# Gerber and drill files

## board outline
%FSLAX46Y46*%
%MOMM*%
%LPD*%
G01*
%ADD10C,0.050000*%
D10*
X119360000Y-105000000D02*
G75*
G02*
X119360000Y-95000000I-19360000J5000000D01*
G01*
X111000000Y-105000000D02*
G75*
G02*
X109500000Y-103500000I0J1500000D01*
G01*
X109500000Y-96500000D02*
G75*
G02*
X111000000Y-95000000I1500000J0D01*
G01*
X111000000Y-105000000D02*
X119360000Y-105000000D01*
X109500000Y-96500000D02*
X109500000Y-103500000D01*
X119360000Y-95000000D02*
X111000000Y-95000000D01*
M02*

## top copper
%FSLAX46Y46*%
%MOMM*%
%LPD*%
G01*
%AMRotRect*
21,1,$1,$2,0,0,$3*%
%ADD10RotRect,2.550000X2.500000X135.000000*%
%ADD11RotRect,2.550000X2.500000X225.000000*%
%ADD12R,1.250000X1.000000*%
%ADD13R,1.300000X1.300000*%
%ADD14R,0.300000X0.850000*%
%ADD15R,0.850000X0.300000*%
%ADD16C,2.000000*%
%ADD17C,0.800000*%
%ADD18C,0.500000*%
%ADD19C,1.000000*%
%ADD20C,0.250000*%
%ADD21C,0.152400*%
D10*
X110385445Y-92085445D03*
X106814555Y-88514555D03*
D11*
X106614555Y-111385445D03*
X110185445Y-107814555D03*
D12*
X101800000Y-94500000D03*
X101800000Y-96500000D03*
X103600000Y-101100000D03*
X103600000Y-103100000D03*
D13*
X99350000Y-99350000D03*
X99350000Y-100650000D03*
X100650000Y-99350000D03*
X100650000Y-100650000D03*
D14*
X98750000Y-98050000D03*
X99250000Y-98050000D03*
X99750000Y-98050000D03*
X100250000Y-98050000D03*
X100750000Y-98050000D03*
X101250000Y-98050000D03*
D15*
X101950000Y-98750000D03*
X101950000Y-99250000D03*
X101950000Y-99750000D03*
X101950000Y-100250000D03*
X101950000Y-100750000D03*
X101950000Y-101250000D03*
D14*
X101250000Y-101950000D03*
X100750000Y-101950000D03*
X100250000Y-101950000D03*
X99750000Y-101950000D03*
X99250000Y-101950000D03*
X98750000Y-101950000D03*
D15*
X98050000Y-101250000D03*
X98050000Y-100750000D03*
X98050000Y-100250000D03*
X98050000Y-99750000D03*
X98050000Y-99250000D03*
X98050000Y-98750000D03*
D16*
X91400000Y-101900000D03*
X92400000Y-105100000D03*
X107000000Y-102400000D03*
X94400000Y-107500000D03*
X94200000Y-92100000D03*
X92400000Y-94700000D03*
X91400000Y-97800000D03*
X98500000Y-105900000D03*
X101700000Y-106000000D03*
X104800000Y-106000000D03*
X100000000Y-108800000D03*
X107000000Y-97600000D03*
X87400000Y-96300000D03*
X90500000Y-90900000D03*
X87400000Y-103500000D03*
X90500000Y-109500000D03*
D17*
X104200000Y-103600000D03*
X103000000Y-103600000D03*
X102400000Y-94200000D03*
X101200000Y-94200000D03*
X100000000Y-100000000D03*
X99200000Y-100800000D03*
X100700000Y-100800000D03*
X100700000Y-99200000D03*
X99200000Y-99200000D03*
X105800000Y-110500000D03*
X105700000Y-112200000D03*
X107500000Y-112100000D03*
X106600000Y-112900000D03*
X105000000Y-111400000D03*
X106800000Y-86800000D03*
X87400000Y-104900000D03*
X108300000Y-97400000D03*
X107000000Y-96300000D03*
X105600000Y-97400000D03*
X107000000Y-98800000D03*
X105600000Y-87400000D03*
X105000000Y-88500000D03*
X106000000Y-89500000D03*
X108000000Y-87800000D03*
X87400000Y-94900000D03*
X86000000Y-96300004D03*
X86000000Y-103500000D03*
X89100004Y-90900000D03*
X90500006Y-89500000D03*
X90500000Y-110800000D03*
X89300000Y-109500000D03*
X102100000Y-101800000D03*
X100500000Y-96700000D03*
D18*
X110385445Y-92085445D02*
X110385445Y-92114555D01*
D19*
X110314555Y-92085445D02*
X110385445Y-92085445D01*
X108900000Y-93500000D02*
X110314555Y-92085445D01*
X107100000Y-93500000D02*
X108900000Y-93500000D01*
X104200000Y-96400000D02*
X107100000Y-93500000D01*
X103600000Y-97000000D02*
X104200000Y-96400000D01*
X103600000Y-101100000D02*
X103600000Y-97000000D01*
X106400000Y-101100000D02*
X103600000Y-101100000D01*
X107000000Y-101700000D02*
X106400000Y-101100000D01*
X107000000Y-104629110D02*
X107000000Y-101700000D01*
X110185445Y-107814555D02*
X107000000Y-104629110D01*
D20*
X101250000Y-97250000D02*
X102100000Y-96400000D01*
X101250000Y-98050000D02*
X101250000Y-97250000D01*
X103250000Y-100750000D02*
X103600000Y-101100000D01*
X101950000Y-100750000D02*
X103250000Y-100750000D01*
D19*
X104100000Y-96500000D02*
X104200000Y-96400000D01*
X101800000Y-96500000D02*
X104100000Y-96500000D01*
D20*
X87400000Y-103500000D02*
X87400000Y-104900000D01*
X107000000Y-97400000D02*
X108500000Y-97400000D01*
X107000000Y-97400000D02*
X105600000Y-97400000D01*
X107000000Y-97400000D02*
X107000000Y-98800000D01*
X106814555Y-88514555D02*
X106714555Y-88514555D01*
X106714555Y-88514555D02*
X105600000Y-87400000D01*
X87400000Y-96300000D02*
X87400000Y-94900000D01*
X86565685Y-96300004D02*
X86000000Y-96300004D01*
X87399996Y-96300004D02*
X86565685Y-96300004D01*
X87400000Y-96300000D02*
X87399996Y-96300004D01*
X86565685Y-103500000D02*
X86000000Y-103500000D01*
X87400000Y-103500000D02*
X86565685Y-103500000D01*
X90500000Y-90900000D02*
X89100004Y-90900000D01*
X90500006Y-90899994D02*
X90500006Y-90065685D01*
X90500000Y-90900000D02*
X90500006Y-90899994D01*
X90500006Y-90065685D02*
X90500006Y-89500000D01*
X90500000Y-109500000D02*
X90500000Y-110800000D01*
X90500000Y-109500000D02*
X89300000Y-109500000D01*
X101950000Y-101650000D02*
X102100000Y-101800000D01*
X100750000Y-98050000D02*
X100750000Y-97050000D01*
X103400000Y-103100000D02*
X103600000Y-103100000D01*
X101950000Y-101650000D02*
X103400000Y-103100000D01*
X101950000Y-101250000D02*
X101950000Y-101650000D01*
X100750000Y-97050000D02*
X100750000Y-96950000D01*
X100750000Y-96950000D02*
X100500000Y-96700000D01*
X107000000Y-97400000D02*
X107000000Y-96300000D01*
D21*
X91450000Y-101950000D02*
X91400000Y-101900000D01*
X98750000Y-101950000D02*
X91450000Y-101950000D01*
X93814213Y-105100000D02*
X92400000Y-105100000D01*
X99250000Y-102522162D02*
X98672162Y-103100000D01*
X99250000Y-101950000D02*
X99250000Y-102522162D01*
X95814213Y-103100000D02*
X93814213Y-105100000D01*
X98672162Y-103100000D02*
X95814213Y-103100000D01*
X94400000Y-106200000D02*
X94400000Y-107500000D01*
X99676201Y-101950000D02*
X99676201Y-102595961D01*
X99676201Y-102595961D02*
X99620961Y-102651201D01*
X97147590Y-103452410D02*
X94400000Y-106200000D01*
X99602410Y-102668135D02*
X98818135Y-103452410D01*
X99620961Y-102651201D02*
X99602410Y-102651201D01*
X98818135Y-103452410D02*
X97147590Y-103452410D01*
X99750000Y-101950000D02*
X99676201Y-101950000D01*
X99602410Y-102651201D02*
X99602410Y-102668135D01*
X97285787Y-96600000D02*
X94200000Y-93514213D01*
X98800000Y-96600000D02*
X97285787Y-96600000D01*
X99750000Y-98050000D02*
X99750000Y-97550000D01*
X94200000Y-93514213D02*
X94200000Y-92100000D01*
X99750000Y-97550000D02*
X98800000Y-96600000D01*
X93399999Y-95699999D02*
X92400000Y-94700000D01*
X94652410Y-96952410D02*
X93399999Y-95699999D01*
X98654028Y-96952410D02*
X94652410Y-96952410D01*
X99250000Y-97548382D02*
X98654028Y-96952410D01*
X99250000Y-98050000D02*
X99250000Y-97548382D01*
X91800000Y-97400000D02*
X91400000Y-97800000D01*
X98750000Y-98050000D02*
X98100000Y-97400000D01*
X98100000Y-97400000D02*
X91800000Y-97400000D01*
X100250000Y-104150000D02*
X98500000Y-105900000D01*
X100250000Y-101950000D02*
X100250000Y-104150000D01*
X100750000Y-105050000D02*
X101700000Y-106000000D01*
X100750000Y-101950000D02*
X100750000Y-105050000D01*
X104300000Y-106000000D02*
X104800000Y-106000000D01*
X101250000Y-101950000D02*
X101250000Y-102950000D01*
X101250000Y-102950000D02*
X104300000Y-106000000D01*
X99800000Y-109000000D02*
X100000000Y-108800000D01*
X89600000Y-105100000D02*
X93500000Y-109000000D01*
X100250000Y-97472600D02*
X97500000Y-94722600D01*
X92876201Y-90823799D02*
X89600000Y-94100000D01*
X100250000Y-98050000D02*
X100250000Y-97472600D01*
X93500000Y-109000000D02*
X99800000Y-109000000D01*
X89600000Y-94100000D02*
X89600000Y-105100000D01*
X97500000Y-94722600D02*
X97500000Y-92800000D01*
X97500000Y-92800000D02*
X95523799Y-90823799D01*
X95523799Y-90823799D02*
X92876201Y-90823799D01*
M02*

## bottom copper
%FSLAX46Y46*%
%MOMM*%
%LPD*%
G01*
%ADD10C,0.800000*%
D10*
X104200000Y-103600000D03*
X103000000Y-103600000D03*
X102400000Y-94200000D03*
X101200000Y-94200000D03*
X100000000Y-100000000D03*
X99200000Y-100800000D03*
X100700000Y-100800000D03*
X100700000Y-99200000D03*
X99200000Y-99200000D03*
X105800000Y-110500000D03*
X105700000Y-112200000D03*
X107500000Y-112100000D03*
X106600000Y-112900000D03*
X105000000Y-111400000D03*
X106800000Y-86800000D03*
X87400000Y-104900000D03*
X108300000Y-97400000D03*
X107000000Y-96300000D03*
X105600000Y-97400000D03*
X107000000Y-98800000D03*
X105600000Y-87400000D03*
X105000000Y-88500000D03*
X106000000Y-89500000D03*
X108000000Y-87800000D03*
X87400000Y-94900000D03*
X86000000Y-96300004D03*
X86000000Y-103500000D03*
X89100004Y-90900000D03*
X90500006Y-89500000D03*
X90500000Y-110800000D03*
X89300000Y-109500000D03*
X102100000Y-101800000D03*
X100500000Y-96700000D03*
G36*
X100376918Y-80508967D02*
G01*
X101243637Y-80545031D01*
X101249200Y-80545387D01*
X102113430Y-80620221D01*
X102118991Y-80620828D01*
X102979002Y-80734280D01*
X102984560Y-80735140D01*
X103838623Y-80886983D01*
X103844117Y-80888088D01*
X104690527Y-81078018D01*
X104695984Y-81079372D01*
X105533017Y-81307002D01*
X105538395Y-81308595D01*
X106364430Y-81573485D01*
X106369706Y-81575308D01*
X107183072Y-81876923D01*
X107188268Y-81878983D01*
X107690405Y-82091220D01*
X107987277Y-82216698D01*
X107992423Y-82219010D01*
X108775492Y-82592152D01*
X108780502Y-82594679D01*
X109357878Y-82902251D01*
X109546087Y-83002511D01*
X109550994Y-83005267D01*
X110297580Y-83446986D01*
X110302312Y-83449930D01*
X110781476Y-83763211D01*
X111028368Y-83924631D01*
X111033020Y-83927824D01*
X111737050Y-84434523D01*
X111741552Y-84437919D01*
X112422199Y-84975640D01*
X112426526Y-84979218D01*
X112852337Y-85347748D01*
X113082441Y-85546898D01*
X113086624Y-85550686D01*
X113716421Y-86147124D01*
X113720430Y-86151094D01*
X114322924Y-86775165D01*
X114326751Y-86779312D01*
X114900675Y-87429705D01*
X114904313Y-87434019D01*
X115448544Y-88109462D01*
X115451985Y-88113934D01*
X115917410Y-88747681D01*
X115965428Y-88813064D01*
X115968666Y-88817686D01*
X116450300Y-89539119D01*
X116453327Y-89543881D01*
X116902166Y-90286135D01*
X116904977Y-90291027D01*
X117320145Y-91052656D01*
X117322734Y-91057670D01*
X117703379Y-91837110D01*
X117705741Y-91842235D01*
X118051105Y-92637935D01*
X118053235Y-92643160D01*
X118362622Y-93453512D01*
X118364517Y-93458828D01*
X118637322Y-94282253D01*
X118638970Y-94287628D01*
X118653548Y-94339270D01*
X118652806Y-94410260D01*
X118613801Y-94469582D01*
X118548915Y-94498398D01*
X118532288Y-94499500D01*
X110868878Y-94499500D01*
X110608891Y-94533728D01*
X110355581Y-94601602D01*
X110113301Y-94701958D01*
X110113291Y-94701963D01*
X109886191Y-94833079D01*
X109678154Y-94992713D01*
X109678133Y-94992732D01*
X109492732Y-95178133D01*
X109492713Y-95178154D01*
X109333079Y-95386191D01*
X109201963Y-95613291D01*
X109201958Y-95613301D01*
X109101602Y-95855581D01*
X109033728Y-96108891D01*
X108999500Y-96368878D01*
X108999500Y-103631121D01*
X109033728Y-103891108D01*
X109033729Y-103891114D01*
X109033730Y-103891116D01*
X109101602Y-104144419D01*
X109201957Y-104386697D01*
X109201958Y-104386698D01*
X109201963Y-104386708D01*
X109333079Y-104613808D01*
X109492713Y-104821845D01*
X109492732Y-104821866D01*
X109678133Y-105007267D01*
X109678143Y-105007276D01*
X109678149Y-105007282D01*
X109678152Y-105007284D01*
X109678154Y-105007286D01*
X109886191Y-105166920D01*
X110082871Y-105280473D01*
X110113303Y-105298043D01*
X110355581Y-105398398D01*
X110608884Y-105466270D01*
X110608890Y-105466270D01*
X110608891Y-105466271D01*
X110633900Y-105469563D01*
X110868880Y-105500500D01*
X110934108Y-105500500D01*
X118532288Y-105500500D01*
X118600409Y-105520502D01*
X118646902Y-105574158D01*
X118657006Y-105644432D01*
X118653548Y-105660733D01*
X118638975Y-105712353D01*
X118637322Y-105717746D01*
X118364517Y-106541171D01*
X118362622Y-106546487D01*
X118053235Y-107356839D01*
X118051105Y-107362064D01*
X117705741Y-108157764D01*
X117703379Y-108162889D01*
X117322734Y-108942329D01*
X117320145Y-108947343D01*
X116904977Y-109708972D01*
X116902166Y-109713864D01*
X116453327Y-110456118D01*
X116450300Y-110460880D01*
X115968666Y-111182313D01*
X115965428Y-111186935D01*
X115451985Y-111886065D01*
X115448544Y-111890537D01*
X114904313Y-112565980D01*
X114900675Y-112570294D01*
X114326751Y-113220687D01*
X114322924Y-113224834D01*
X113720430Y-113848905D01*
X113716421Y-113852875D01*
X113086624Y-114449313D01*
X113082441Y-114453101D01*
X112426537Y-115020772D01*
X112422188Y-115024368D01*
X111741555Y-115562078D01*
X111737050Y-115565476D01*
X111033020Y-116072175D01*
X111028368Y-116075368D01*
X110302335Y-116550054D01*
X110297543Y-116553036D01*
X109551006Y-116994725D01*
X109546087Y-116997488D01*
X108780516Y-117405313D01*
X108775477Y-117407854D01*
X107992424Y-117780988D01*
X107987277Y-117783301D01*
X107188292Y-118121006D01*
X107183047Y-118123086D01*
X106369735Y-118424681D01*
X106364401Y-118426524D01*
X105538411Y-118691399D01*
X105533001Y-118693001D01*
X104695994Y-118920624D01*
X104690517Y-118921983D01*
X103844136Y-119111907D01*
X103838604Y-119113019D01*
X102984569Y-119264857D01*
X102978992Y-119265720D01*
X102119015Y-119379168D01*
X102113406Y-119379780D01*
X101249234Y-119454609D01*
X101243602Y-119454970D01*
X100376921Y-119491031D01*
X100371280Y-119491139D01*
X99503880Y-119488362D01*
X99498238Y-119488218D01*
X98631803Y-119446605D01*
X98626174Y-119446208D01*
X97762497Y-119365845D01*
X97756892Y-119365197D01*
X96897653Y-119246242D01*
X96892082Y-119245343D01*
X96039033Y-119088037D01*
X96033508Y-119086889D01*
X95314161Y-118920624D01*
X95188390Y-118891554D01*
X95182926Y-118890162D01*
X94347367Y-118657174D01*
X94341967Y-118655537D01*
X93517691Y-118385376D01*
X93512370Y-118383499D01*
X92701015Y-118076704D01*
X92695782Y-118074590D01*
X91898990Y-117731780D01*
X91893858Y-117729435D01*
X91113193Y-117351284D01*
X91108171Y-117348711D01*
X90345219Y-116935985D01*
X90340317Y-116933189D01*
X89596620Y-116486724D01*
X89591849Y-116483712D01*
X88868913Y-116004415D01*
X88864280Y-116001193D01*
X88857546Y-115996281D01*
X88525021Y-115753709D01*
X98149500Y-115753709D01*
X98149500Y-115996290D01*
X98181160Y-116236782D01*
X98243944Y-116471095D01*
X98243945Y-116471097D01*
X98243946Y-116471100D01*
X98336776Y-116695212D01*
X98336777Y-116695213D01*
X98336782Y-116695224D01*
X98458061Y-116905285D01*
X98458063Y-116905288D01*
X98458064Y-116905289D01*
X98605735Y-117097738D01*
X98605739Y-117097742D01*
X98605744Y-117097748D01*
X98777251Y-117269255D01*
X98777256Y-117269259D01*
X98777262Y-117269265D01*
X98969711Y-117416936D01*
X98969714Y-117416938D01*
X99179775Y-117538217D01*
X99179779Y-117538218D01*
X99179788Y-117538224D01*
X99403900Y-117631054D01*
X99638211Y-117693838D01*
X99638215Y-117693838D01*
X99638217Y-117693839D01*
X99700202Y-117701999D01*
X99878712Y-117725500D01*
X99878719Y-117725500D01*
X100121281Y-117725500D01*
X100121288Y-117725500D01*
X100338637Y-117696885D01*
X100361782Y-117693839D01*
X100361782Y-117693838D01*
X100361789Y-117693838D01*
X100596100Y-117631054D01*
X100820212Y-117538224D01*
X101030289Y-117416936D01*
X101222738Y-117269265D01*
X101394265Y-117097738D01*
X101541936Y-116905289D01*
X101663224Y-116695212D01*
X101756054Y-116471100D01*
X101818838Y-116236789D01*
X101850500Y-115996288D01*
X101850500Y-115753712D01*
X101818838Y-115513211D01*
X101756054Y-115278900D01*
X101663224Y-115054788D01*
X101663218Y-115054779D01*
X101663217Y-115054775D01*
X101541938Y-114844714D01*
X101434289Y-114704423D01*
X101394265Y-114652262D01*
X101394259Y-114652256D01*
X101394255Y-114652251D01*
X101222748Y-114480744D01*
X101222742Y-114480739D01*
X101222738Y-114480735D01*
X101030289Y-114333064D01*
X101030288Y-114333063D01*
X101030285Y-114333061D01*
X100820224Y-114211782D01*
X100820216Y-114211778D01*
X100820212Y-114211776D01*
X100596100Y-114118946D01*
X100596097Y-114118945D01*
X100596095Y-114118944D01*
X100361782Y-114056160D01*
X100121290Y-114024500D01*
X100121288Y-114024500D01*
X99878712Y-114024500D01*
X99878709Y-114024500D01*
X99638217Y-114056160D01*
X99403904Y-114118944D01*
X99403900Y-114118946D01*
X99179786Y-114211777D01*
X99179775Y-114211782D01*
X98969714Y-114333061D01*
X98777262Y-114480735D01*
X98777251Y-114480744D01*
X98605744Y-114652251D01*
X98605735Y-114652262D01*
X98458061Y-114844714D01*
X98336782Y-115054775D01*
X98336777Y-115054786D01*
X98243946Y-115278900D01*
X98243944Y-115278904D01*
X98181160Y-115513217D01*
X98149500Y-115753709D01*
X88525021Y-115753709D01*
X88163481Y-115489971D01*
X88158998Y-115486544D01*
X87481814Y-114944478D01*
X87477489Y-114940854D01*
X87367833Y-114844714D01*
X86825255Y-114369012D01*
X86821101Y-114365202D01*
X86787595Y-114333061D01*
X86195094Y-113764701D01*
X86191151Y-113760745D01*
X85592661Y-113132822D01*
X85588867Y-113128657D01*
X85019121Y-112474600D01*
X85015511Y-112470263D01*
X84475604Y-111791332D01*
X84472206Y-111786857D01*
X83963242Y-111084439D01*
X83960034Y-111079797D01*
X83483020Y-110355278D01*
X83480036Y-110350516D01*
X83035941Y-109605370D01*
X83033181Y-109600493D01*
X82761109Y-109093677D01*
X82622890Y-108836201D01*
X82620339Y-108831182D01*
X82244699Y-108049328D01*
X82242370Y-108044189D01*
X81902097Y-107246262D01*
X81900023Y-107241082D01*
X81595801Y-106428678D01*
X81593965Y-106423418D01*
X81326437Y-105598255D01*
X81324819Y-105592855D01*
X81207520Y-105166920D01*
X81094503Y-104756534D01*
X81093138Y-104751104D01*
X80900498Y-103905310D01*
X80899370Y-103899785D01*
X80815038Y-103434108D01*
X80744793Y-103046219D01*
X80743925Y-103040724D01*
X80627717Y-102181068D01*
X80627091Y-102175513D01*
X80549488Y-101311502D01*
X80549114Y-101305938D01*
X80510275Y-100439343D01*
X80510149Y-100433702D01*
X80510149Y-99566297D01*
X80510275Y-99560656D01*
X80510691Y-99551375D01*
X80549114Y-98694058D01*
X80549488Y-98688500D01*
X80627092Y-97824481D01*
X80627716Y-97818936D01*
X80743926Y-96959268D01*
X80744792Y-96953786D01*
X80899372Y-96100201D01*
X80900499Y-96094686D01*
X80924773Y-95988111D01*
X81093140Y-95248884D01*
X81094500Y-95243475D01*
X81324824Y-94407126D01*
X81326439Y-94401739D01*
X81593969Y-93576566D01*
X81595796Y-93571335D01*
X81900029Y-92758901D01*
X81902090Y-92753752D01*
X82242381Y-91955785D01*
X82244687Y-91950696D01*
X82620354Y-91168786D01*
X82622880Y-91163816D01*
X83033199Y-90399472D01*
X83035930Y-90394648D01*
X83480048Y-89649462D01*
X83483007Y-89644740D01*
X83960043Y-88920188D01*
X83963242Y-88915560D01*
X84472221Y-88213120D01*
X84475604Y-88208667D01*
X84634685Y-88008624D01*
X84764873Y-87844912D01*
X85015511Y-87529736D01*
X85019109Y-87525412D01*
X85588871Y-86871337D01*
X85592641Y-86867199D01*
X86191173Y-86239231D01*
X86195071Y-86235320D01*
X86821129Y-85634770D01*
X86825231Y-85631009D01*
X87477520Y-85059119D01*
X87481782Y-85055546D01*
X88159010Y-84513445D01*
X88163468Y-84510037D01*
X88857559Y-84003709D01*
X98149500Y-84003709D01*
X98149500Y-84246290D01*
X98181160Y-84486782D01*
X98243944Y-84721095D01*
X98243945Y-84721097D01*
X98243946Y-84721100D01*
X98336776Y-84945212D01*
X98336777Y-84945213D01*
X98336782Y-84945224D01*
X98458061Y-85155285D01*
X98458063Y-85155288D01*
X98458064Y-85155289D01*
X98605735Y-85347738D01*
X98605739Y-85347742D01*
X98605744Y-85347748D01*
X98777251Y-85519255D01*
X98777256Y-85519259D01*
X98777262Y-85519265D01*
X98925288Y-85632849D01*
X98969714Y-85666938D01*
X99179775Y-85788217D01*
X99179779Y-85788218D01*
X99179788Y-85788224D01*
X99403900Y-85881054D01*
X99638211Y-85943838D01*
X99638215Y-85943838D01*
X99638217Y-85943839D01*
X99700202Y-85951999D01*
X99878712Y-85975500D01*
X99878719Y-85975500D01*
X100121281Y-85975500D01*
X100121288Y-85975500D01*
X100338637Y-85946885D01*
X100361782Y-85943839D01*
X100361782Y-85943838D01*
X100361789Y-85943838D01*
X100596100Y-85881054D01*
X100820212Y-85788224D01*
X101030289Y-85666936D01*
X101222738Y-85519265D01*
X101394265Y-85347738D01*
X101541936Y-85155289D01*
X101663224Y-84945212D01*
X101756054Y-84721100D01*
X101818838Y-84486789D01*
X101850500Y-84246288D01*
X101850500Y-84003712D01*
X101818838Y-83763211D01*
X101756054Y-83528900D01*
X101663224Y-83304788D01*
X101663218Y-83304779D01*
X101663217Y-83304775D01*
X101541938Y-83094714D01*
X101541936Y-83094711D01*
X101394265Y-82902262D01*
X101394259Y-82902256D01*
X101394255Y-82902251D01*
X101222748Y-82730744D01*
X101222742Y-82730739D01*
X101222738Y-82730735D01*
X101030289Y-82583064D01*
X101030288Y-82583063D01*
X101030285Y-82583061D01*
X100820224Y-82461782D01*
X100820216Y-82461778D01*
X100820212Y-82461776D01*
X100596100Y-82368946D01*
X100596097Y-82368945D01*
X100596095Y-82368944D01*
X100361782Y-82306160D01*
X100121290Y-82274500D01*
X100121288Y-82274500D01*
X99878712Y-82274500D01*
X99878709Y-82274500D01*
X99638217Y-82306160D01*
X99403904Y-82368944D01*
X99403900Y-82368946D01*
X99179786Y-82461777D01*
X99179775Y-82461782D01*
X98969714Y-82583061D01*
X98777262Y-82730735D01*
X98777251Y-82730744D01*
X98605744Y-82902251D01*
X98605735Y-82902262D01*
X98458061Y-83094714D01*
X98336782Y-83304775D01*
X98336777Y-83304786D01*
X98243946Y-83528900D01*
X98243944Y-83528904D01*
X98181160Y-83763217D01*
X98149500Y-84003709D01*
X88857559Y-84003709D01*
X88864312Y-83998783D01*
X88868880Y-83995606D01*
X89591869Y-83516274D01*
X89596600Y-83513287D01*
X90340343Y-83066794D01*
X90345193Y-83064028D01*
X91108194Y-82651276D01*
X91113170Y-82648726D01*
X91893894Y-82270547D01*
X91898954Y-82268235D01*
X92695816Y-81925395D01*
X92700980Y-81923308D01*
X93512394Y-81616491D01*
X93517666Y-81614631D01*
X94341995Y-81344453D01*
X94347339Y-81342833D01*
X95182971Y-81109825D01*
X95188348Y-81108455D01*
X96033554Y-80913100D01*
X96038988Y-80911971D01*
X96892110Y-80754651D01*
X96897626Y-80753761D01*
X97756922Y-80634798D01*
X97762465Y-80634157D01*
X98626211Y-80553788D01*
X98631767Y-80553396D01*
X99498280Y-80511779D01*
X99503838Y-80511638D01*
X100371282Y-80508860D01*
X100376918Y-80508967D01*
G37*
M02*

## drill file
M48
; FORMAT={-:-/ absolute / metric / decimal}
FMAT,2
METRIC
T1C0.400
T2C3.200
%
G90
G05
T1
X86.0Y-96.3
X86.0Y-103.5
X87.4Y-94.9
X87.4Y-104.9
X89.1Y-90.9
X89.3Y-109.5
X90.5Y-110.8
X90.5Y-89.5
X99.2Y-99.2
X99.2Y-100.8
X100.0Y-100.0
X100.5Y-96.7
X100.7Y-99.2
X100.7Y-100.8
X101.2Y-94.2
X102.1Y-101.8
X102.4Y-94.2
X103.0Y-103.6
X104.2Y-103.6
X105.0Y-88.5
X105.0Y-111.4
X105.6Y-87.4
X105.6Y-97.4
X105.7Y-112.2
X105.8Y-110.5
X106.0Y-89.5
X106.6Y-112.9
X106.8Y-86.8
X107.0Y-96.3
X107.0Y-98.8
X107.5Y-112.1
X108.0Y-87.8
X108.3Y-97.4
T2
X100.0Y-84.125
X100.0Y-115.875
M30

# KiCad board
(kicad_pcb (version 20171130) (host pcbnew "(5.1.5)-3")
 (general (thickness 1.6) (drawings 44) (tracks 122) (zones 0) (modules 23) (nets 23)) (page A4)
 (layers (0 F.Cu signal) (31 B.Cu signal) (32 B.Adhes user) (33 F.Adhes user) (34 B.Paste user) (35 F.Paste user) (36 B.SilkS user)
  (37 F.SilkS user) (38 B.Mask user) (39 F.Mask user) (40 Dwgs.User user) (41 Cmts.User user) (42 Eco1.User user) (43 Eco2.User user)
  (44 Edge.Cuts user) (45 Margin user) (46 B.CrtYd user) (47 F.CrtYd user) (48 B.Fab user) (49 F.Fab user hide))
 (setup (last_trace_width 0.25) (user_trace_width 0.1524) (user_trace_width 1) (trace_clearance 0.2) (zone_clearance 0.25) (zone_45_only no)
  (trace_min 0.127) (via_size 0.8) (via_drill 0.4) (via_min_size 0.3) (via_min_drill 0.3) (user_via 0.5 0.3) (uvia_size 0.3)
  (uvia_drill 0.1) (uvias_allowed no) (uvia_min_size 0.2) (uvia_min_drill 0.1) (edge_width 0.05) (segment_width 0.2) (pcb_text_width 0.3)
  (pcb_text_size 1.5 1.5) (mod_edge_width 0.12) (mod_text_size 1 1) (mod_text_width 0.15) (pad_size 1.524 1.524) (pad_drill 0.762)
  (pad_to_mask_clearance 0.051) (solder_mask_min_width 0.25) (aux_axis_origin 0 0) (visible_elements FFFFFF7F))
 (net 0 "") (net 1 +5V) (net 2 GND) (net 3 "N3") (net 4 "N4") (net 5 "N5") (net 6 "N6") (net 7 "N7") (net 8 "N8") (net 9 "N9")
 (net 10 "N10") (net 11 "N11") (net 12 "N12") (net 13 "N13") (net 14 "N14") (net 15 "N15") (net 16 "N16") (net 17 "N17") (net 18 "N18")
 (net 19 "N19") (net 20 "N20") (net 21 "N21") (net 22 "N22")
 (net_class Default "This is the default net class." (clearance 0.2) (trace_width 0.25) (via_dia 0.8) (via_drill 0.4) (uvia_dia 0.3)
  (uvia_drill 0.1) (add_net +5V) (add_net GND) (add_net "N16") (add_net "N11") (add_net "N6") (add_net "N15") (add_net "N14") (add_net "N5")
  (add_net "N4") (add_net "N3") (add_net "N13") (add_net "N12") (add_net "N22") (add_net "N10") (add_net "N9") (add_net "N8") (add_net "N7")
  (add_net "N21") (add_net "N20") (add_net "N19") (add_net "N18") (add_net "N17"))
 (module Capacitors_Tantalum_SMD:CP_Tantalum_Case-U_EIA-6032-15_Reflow (layer F.Cu) (at 108.6 90.3 135)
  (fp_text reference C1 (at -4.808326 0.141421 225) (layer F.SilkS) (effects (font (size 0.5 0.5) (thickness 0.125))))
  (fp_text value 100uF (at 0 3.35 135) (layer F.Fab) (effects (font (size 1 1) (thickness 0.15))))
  (pad 1 smd rect (at -2.525 0 135) (size 2.55 2.5) (layers F.Cu F.Paste F.Mask) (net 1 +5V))
  (pad 2 smd rect (at 2.525 0 135) (size 2.55 2.5) (layers F.Cu F.Paste F.Mask) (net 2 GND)))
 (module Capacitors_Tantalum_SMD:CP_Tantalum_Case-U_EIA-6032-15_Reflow (layer F.Cu) (at 108.4 109.6 225)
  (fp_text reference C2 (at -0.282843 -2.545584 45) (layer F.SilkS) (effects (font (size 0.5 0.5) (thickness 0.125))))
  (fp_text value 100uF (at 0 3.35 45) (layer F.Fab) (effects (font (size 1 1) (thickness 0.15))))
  (pad 2 smd rect (at 2.525 0 225) (size 2.55 2.5) (layers F.Cu F.Paste F.Mask) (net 2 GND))
  (pad 1 smd rect (at -2.525 0 225) (size 2.55 2.5) (layers F.Cu F.Paste F.Mask) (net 1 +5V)))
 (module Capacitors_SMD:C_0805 (layer F.Cu) (at 101.8 95.5 90)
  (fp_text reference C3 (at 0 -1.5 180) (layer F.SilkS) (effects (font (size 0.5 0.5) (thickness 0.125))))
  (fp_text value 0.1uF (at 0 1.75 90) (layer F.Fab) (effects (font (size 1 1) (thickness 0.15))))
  (pad 2 smd rect (at 1 0 90) (size 1 1.25) (layers F.Cu F.Paste F.Mask) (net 2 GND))
  (pad 1 smd rect (at -1 0 90) (size 1 1.25) (layers F.Cu F.Paste F.Mask) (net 1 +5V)))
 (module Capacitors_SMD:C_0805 (layer F.Cu) (at 103.6 102.1 270)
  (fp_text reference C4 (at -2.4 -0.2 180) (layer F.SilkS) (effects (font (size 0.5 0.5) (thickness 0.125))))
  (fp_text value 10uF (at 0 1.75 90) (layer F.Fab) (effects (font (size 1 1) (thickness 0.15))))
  (pad 1 smd rect (at -1 0 270) (size 1 1.25) (layers F.Cu F.Paste F.Mask) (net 1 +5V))
  (pad 2 smd rect (at 1 0 270) (size 1 1.25) (layers F.Cu F.Paste F.Mask) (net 2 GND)))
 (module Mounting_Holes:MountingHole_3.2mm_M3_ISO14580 (layer F.Cu) (at 100 84.125)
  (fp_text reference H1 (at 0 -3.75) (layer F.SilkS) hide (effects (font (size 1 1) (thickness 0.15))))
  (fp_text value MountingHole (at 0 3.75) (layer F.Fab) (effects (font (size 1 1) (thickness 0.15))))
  (pad 1 np_thru_hole circle (at 0 0) (size 3.2 3.2) (drill 3.2) (layers *.Cu *.Mask)))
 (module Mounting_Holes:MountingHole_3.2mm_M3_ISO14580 (layer F.Cu) (at 100 115.875)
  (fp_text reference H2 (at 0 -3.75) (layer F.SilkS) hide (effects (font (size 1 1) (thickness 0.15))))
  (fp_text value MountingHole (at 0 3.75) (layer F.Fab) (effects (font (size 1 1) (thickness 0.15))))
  (pad 1 np_thru_hole circle (at 0 0) (size 3.2 3.2) (drill 3.2) (layers *.Cu *.Mask)))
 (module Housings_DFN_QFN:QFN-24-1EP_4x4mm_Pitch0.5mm (layer F.Cu) (at 100 100) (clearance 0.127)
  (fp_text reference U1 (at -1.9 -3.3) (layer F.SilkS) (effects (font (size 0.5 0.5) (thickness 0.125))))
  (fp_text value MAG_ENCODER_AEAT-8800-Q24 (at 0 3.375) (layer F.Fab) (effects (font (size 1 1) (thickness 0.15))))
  (pad 25 smd rect (at -0.65 -0.65) (size 1.3 1.3) (layers F.Cu F.Paste F.Mask) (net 2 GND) (solder_paste_margin_ratio -0.2))
  (pad 25 smd rect (at -0.65 0.65) (size 1.3 1.3) (layers F.Cu F.Paste F.Mask) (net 2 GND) (solder_paste_margin_ratio -0.2))
  (pad 25 smd rect (at 0.65 -0.65) (size 1.3 1.3) (layers F.Cu F.Paste F.Mask) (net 2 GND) (solder_paste_margin_ratio -0.2))
  (pad 25 smd rect (at 0.65 0.65) (size 1.3 1.3) (layers F.Cu F.Paste F.Mask) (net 2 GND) (solder_paste_margin_ratio -0.2))
  (pad 24 smd rect (at -1.25 -1.95 90) (size 0.85 0.3) (layers F.Cu F.Paste F.Mask) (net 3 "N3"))
  (pad 23 smd rect (at -0.75 -1.95 90) (size 0.85 0.3) (layers F.Cu F.Paste F.Mask) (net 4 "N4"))
  (pad 22 smd rect (at -0.25 -1.95 90) (size 0.85 0.3) (layers F.Cu F.Paste F.Mask) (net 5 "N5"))
  (pad 21 smd rect (at 0.25 -1.95 90) (size 0.85 0.3) (layers F.Cu F.Paste F.Mask) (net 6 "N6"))
  (pad 20 smd rect (at 0.75 -1.95 90) (size 0.85 0.3) (layers F.Cu F.Paste F.Mask) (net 2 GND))
  (pad 19 smd rect (at 1.25 -1.95 90) (size 0.85 0.3) (layers F.Cu F.Paste F.Mask) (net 1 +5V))
  (pad 18 smd rect (at 1.95 -1.25) (size 0.85 0.3) (layers F.Cu F.Paste F.Mask) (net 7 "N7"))
  (pad 17 smd rect (at 1.95 -0.75) (size 0.85 0.3) (layers F.Cu F.Paste F.Mask) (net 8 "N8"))
  (pad 16 smd rect (at 1.95 -0.25) (size 0.85 0.3) (layers F.Cu F.Paste F.Mask) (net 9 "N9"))
  (pad 15 smd rect (at 1.95 0.25) (size 0.85 0.3) (layers F.Cu F.Paste F.Mask) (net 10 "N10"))
  (pad 14 smd rect (at 1.95 0.75) (size 0.85 0.3) (layers F.Cu F.Paste F.Mask) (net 1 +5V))
  (pad 13 smd rect (at 1.95 1.25) (size 0.85 0.3) (layers F.Cu F.Paste F.Mask) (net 2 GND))
  (pad 12 smd rect (at 1.25 1.95 90) (size 0.85 0.3) (layers F.Cu F.Paste F.Mask) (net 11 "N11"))
  (pad 11 smd rect (at 0.75 1.95 90) (size 0.85 0.3) (layers F.Cu F.Paste F.Mask) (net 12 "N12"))
  (pad 10 smd rect (at 0.25 1.95 90) (size 0.85 0.3) (layers F.Cu F.Paste F.Mask) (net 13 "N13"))
  (pad 9 smd rect (at -0.25 1.95 90) (size 0.85 0.3) (layers F.Cu F.Paste F.Mask) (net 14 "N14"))
  (pad 8 smd rect (at -0.75 1.95 90) (size 0.85 0.3) (layers F.Cu F.Paste F.Mask) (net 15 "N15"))
  (pad 7 smd rect (at -1.25 1.95 90) (size 0.85 0.3) (layers F.Cu F.Paste F.Mask) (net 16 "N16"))
  (pad 6 smd rect (at -1.95 1.25) (size 0.85 0.3) (layers F.Cu F.Paste F.Mask) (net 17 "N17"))
  (pad 5 smd rect (at -1.95 0.75) (size 0.85 0.3) (layers F.Cu F.Paste F.Mask) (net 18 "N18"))
  (pad 4 smd rect (at -1.95 0.25) (size 0.85 0.3) (layers F.Cu F.Paste F.Mask) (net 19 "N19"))
  (pad 3 smd rect (at -1.95 -0.25) (size 0.85 0.3) (layers F.Cu F.Paste F.Mask) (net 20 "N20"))
  (pad 2 smd rect (at -1.95 -0.75) (size 0.85 0.3) (layers F.Cu F.Paste F.Mask) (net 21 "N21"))
  (pad 1 smd rect (at -1.95 -1.25) (size 0.85 0.3) (layers F.Cu F.Paste F.Mask) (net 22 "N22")))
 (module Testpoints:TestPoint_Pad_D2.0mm (layer F.Cu) (at 91.4 101.9)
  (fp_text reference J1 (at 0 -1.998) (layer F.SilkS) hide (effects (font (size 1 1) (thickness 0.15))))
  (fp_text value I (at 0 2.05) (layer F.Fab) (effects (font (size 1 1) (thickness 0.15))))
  (pad 1 smd circle (at 0 0) (size 2 2) (layers F.Cu F.Mask) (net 16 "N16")))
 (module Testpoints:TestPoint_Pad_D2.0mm (layer F.Cu) (at 92.4 105.1)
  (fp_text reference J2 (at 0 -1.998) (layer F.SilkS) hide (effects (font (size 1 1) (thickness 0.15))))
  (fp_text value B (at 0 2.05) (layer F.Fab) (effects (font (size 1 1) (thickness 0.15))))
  (pad 1 smd circle (at 0 0) (size 2 2) (layers F.Cu F.Mask) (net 15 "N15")))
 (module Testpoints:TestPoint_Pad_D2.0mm (layer F.Cu) (at 107 102.4)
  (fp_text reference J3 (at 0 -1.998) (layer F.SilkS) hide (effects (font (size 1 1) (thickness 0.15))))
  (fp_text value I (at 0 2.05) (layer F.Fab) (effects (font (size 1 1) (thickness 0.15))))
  (pad 1 smd circle (at 0 0) (size 2 2) (layers F.Cu F.Mask) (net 1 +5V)))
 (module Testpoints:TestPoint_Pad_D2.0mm (layer F.Cu) (at 94.4 107.5)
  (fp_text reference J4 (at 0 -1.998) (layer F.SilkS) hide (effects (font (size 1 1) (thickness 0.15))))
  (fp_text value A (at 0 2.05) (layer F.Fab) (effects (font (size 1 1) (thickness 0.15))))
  (pad 1 smd circle (at 0 0) (size 2 2) (layers F.Cu F.Mask) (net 14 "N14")))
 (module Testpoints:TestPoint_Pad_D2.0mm (layer F.Cu) (at 94.2 92.1)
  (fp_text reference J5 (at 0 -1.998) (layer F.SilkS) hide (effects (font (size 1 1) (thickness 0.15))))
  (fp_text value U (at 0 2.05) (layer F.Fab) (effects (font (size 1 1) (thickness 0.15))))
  (pad 1 smd circle (at 0 0) (size 2 2) (layers F.Cu F.Mask) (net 5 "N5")))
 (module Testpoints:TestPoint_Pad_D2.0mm (layer F.Cu) (at 92.4 94.7)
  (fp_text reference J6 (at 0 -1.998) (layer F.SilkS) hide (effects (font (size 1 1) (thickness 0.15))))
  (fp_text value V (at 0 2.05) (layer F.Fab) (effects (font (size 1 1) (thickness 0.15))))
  (pad 1 smd circle (at 0 0) (size 2 2) (layers F.Cu F.Mask) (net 4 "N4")))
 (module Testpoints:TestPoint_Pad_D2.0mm (layer F.Cu) (at 91.4 97.8)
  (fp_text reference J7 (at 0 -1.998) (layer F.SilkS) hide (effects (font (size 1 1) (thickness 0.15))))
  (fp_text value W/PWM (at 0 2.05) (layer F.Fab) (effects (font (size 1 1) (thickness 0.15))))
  (pad 1 smd circle (at 0 0) (size 2 2) (layers F.Cu F.Mask) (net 3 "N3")))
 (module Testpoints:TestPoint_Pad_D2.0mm (layer F.Cu) (at 98.5 105.9)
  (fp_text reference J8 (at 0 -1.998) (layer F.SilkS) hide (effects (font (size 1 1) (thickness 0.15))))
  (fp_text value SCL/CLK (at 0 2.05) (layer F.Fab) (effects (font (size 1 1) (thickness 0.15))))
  (pad 1 smd circle (at 0 0) (size 2 2) (layers F.Cu F.Mask) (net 13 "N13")))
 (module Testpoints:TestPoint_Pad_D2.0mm (layer F.Cu) (at 101.7 106)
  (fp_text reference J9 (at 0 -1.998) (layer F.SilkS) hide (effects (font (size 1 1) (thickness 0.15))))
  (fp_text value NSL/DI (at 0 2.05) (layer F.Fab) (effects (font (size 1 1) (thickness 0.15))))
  (pad 1 smd circle (at 0 0) (size 2 2) (layers F.Cu F.Mask) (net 12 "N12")))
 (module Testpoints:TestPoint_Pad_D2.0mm (layer F.Cu) (at 104.8 106)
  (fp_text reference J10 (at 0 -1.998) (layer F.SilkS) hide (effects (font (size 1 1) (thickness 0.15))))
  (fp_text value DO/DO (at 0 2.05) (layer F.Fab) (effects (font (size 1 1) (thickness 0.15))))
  (pad 1 smd circle (at 0 0) (size 2 2) (layers F.Cu F.Mask) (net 11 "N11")))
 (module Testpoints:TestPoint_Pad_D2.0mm (layer F.Cu) (at 100 108.8)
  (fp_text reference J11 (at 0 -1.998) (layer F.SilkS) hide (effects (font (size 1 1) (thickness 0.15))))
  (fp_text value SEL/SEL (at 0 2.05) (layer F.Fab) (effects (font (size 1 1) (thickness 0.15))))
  (pad 1 smd circle (at 0 0) (size 2 2) (layers F.Cu F.Mask) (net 6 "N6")))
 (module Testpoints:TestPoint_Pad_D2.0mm (layer F.Cu) (at 107 97.6)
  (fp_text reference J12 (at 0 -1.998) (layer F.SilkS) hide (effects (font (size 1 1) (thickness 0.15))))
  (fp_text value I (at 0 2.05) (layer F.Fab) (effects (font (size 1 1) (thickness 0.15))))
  (pad 1 smd circle (at 0 0) (size 2 2) (layers F.Cu F.Mask) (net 2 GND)))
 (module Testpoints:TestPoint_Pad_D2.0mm (layer F.Cu) (at 87.4 96.3)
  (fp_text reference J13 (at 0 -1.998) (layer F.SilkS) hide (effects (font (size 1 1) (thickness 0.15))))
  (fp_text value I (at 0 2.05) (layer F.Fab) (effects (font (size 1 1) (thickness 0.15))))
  (pad 1 smd circle (at 0 0) (size 2 2) (layers F.Cu F.Mask) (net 2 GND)))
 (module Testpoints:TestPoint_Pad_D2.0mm (layer F.Cu) (at 90.5 90.9)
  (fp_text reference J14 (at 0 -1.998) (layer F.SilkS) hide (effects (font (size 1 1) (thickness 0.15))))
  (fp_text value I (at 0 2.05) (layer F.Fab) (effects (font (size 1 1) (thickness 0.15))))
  (pad 1 smd circle (at 0 0) (size 2 2) (layers F.Cu F.Mask) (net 2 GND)))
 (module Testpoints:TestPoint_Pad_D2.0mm (layer F.Cu) (at 87.4 103.5)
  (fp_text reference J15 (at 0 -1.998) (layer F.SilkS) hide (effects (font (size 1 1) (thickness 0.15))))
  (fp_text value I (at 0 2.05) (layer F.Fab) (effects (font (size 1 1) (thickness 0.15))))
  (pad 1 smd circle (at 0 0) (size 2 2) (layers F.Cu F.Mask) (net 2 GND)))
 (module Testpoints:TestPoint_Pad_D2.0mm (layer F.Cu) (at 90.5 109.5)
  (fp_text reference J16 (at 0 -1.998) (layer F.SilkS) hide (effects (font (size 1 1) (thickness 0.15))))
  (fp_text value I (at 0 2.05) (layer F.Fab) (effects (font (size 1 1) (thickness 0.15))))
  (pad 1 smd circle (at 0 0) (size 2 2) (layers F.Cu F.Mask) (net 2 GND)))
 (gr_arc (start 100 100) (end 119.36 95) (angle -331.0379313) (layer Edge.Cuts) (width 0.05))
 (gr_arc (start 111 103.5) (end 109.5 103.5) (angle -90) (layer Edge.Cuts) (width 0.05))
 (gr_arc (start 111 96.5) (end 111 95) (angle -90) (layer Edge.Cuts) (width 0.05))
 (gr_line (start 111 105) (end 119.36 105) (layer Edge.Cuts) (width 0.05))
 (gr_line (start 109.5 96.5) (end 109.5 103.5) (layer Edge.Cuts) (width 0.05))
 (gr_line (start 119.36 95) (end 111 95) (layer Edge.Cuts) (width 0.05))
 (via (at 104.2 103.6) (size 0.8) (drill 0.4) (layers F.Cu B.Cu) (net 2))
 (via (at 103 103.6) (size 0.8) (drill 0.4) (layers F.Cu B.Cu) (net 2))
 (via (at 102.4 94.2) (size 0.8) (drill 0.4) (layers F.Cu B.Cu) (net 2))
 (via (at 101.2 94.2) (size 0.8) (drill 0.4) (layers F.Cu B.Cu) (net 2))
 (via (at 100 100) (size 0.8) (drill 0.4) (layers F.Cu B.Cu) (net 2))
 (via (at 99.2 100.8) (size 0.8) (drill 0.4) (layers F.Cu B.Cu) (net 2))
 (via (at 100.7 100.8) (size 0.8) (drill 0.4) (layers F.Cu B.Cu) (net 2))
 (via (at 100.7 99.2) (size 0.8) (drill 0.4) (layers F.Cu B.Cu) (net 2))
 (via (at 99.2 99.2) (size 0.8) (drill 0.4) (layers F.Cu B.Cu) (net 2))
 (segment (start 110.385445 92.085445) (end 110.385445 92.114555) (width 0.5) (layer F.Cu) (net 1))
 (segment (start 110.314555 92.085445) (end 110.385445 92.085445) (width 1) (layer F.Cu) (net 1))
 (segment (start 108.9 93.5) (end 110.314555 92.085445) (width 1) (layer F.Cu) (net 1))
 (segment (start 107.1 93.5) (end 108.9 93.5) (width 1) (layer F.Cu) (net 1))
 (segment (start 104.2 96.4) (end 107.1 93.5) (width 1) (layer F.Cu) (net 1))
 (segment (start 103.6 97) (end 104.2 96.4) (width 1) (layer F.Cu) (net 1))
 (segment (start 103.6 101.1) (end 103.6 97) (width 1) (layer F.Cu) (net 1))
 (segment (start 106.4 101.1) (end 103.6 101.1) (width 1) (layer F.Cu) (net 1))
 (segment (start 107 101.7) (end 106.4 101.1) (width 1) (layer F.Cu) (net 1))
 (segment (start 107 104.62911) (end 107 101.7) (width 1) (layer F.Cu) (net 1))
 (segment (start 110.185445 107.814555) (end 107 104.62911) (width 1) (layer F.Cu) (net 1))
 (segment (start 101.25 97.25) (end 102.1 96.4) (width 0.25) (layer F.Cu) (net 1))
 (segment (start 101.25 98.05) (end 101.25 97.25) (width 0.25) (layer F.Cu) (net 1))
 (segment (start 103.25 100.75) (end 103.6 101.1) (width 0.25) (layer F.Cu) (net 1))
 (segment (start 101.95 100.75) (end 103.25 100.75) (width 0.25) (layer F.Cu) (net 1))
 (segment (start 104.1 96.5) (end 104.2 96.4) (width 1) (layer F.Cu) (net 1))
 (segment (start 101.8 96.5) (end 104.1 96.5) (width 1) (layer F.Cu) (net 1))
 (via (at 105.8 110.5) (size 0.8) (drill 0.4) (layers F.Cu B.Cu) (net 2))
 (via (at 105.7 112.2) (size 0.8) (drill 0.4) (layers F.Cu B.Cu) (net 2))
 (via (at 107.5 112.1) (size 0.8) (drill 0.4) (layers F.Cu B.Cu) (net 2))
 (via (at 106.6 112.9) (size 0.8) (drill 0.4) (layers F.Cu B.Cu) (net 2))
 (via (at 105 111.4) (size 0.8) (drill 0.4) (layers F.Cu B.Cu) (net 2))
 (via (at 106.8 86.8) (size 0.8) (drill 0.4) (layers F.Cu B.Cu) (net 2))
 (via (at 87.4 104.9) (size 0.8) (drill 0.4) (layers F.Cu B.Cu) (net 2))
 (segment (start 87.4 103.5) (end 87.4 104.9) (width 0.25) (layer F.Cu) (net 2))
 (via (at 108.3 97.4) (size 0.8) (drill 0.4) (layers F.Cu B.Cu) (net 2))
 (segment (start 107 97.4) (end 108.5 97.4) (width 0.25) (layer F.Cu) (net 2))
 (via (at 107 96.3) (size 0.8) (drill 0.4) (layers F.Cu B.Cu) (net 2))
 (via (at 105.6 97.4) (size 0.8) (drill 0.4) (layers F.Cu B.Cu) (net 2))
 (segment (start 107 97.4) (end 105.6 97.4) (width 0.25) (layer F.Cu) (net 2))
 (via (at 107 98.8) (size 0.8) (drill 0.4) (layers F.Cu B.Cu) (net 2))
 (segment (start 107 97.4) (end 107 98.8) (width 0.25) (layer F.Cu) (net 2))
 (via (at 105.6 87.4) (size 0.8) (drill 0.4) (layers F.Cu B.Cu) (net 2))
 (segment (start 106.814555 88.514555) (end 106.714555 88.514555) (width 0.25) (layer F.Cu) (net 2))
 (segment (start 106.714555 88.514555) (end 105.6 87.4) (width 0.25) (layer F.Cu) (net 2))
 (via (at 105 88.5) (size 0.8) (drill 0.4) (layers F.Cu B.Cu) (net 2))
 (via (at 106 89.5) (size 0.8) (drill 0.4) (layers F.Cu B.Cu) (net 2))
 (via (at 108 87.8) (size 0.8) (drill 0.4) (layers F.Cu B.Cu) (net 2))
 (via (at 87.4 94.9) (size 0.8) (drill 0.4) (layers F.Cu B.Cu) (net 2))
 (segment (start 87.4 96.3) (end 87.4 94.9) (width 0.25) (layer F.Cu) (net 2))
 (via (at 86 96.300004) (size 0.8) (drill 0.4) (layers F.Cu B.Cu) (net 2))
 (segment (start 86.565685 96.300004) (end 86 96.300004) (width 0.25) (layer F.Cu) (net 2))
 (segment (start 87.399996 96.300004) (end 86.565685 96.300004) (width 0.25) (layer F.Cu) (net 2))
 (segment (start 87.4 96.3) (end 87.399996 96.300004) (width 0.25) (layer F.Cu) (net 2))
 (segment (start 86.565685 103.5) (end 86 103.5) (width 0.25) (layer F.Cu) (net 2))
 (via (at 86 103.5) (size 0.8) (drill 0.4) (layers F.Cu B.Cu) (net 2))
 (segment (start 87.4 103.5) (end 86.565685 103.5) (width 0.25) (layer F.Cu) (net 2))
 (via (at 89.100004 90.9) (size 0.8) (drill 0.4) (layers F.Cu B.Cu) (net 2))
 (segment (start 90.5 90.9) (end 89.100004 90.9) (width 0.25) (layer F.Cu) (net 2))
 (via (at 90.500006 89.5) (size 0.8) (drill 0.4) (layers F.Cu B.Cu) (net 2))
 (segment (start 90.500006 90.899994) (end 90.500006 90.065685) (width 0.25) (layer F.Cu) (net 2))
 (segment (start 90.5 90.9) (end 90.500006 90.899994) (width 0.25) (layer F.Cu) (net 2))
 (segment (start 90.500006 90.065685) (end 90.500006 89.5) (width 0.25) (layer F.Cu) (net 2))
 (via (at 90.5 110.8) (size 0.8) (drill 0.4) (layers F.Cu B.Cu) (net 2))
 (segment (start 90.5 109.5) (end 90.5 110.8) (width 0.25) (layer F.Cu) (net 2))
 (via (at 89.3 109.5) (size 0.8) (drill 0.4) (layers F.Cu B.Cu) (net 2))
 (segment (start 90.5 109.5) (end 89.3 109.5) (width 0.25) (layer F.Cu) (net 2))
 (via (at 102.1 101.8) (size 0.8) (drill 0.4) (layers F.Cu B.Cu) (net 2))
 (segment (start 101.95 101.65) (end 102.1 101.8) (width 0.25) (layer F.Cu) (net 2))
 (segment (start 100.75 98.05) (end 100.75 97.05) (width 0.25) (layer F.Cu) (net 2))
 (segment (start 103.4 103.1) (end 103.6 103.1) (width 0.25) (layer F.Cu) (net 2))
 (segment (start 101.95 101.65) (end 103.4 103.1) (width 0.25) (layer F.Cu) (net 2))
 (segment (start 101.95 101.25) (end 101.95 101.65) (width 0.25) (layer F.Cu) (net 2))
 (via (at 100.5 96.7) (size 0.8) (drill 0.4) (layers F.Cu B.Cu) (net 2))
 (segment (start 100.75 97.05) (end 100.75 96.95) (width 0.25) (layer F.Cu) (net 2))
 (segment (start 100.75 96.95) (end 100.5 96.7) (width 0.25) (layer F.Cu) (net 2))
 (segment (start 107 97.4) (end 107 96.3) (width 0.25) (layer F.Cu) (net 2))
 (segment (start 91.45 101.95) (end 91.4 101.9) (width 0.1524) (layer F.Cu) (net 16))
 (segment (start 98.75 101.95) (end 91.45 101.95) (width 0.1524) (layer F.Cu) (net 16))
 (segment (start 93.814213 105.1) (end 92.4 105.1) (width 0.1524) (layer F.Cu) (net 15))
 (segment (start 99.25 102.522162) (end 98.672162 103.1) (width 0.1524) (layer F.Cu) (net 15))
 (segment (start 99.25 101.95) (end 99.25 102.522162) (width 0.1524) (layer F.Cu) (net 15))
 (segment (start 95.814213 103.1) (end 93.814213 105.1) (width 0.1524) (layer F.Cu) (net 15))
 (segment (start 98.672162 103.1) (end 95.814213 103.1) (width 0.1524) (layer F.Cu) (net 15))
 (segment (start 94.4 106.2) (end 94.4 107.5) (width 0.1524) (layer F.Cu) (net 14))
 (segment (start 99.676201 101.95) (end 99.676201 102.595961) (width 0.1524) (layer F.Cu) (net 14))
 (segment (start 99.676201 102.595961) (end 99.620961 102.651201) (width 0.1524) (layer F.Cu) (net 14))
 (segment (start 97.14759 103.45241) (end 94.4 106.2) (width 0.1524) (layer F.Cu) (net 14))
 (segment (start 99.60241 102.668135) (end 98.818135 103.45241) (width 0.1524) (layer F.Cu) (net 14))
 (segment (start 99.620961 102.651201) (end 99.60241 102.651201) (width 0.1524) (layer F.Cu) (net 14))
 (segment (start 98.818135 103.45241) (end 97.14759 103.45241) (width 0.1524) (layer F.Cu) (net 14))
 (segment (start 99.75 101.95) (end 99.676201 101.95) (width 0.1524) (layer F.Cu) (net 14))
 (segment (start 99.60241 102.651201) (end 99.60241 102.668135) (width 0.1524) (layer F.Cu) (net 14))
 (segment (start 97.285787 96.6) (end 94.2 93.514213) (width 0.1524) (layer F.Cu) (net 5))
 (segment (start 98.8 96.6) (end 97.285787 96.6) (width 0.1524) (layer F.Cu) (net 5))
 (segment (start 99.75 98.05) (end 99.75 97.55) (width 0.1524) (layer F.Cu) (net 5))
 (segment (start 94.2 93.514213) (end 94.2 92.1) (width 0.1524) (layer F.Cu) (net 5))
 (segment (start 99.75 97.55) (end 98.8 96.6) (width 0.1524) (layer F.Cu) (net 5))
 (segment (start 93.399999 95.699999) (end 92.4 94.7) (width 0.1524) (layer F.Cu) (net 4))
 (segment (start 94.65241 96.95241) (end 93.399999 95.699999) (width 0.1524) (layer F.Cu) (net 4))
 (segment (start 98.654028 96.95241) (end 94.65241 96.95241) (width 0.1524) (layer F.Cu) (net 4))
 (segment (start 99.25 97.548382) (end 98.654028 96.95241) (width 0.1524) (layer F.Cu) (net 4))
 (segment (start 99.25 98.05) (end 99.25 97.548382) (width 0.1524) (layer F.Cu) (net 4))
 (segment (start 91.8 97.4) (end 91.4 97.8) (width 0.1524) (layer F.Cu) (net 3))
 (segment (start 98.75 98.05) (end 98.1 97.4) (width 0.1524) (layer F.Cu) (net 3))
 (segment (start 98.1 97.4) (end 91.8 97.4) (width 0.1524) (layer F.Cu) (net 3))
 (segment (start 100.25 104.15) (end 98.5 105.9) (width 0.1524) (layer F.Cu) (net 13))
 (segment (start 100.25 101.95) (end 100.25 104.15) (width 0.1524) (layer F.Cu) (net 13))
 (segment (start 100.75 105.05) (end 101.7 106) (width 0.1524) (layer F.Cu) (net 12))
 (segment (start 100.75 101.95) (end 100.75 105.05) (width 0.1524) (layer F.Cu) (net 12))
 (segment (start 104.3 106) (end 104.8 106) (width 0.1524) (layer F.Cu) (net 11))
 (segment (start 101.25 101.95) (end 101.25 102.95) (width 0.1524) (layer F.Cu) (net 11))
 (segment (start 101.25 102.95) (end 104.3 106) (width 0.1524) (layer F.Cu) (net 11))
 (segment (start 99.8 109) (end 100 108.8) (width 0.1524) (layer F.Cu) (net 6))
 (segment (start 89.6 105.1) (end 93.5 109) (width 0.1524) (layer F.Cu) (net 6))
 (segment (start 100.25 97.4726) (end 97.5 94.7226) (width 0.1524) (layer F.Cu) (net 6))
 (segment (start 92.876201 90.823799) (end 89.6 94.1) (width 0.1524) (layer F.Cu) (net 6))
 (segment (start 100.25 98.05) (end 100.25 97.4726) (width 0.1524) (layer F.Cu) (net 6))
 (segment (start 93.5 109) (end 99.8 109) (width 0.1524) (layer F.Cu) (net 6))
 (segment (start 89.6 94.1) (end 89.6 105.1) (width 0.1524) (layer F.Cu) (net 6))
 (segment (start 97.5 94.7226) (end 97.5 92.8) (width 0.1524) (layer F.Cu) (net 6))
 (segment (start 97.5 92.8) (end 95.523799 90.823799) (width 0.1524) (layer F.Cu) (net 6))
 (segment (start 95.523799 90.823799) (end 92.876201 90.823799) (width 0.1524) (layer F.Cu) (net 6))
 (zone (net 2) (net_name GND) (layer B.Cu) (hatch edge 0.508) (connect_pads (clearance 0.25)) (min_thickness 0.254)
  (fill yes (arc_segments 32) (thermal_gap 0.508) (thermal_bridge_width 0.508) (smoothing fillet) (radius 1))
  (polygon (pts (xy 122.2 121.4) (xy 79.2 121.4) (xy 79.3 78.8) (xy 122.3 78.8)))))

